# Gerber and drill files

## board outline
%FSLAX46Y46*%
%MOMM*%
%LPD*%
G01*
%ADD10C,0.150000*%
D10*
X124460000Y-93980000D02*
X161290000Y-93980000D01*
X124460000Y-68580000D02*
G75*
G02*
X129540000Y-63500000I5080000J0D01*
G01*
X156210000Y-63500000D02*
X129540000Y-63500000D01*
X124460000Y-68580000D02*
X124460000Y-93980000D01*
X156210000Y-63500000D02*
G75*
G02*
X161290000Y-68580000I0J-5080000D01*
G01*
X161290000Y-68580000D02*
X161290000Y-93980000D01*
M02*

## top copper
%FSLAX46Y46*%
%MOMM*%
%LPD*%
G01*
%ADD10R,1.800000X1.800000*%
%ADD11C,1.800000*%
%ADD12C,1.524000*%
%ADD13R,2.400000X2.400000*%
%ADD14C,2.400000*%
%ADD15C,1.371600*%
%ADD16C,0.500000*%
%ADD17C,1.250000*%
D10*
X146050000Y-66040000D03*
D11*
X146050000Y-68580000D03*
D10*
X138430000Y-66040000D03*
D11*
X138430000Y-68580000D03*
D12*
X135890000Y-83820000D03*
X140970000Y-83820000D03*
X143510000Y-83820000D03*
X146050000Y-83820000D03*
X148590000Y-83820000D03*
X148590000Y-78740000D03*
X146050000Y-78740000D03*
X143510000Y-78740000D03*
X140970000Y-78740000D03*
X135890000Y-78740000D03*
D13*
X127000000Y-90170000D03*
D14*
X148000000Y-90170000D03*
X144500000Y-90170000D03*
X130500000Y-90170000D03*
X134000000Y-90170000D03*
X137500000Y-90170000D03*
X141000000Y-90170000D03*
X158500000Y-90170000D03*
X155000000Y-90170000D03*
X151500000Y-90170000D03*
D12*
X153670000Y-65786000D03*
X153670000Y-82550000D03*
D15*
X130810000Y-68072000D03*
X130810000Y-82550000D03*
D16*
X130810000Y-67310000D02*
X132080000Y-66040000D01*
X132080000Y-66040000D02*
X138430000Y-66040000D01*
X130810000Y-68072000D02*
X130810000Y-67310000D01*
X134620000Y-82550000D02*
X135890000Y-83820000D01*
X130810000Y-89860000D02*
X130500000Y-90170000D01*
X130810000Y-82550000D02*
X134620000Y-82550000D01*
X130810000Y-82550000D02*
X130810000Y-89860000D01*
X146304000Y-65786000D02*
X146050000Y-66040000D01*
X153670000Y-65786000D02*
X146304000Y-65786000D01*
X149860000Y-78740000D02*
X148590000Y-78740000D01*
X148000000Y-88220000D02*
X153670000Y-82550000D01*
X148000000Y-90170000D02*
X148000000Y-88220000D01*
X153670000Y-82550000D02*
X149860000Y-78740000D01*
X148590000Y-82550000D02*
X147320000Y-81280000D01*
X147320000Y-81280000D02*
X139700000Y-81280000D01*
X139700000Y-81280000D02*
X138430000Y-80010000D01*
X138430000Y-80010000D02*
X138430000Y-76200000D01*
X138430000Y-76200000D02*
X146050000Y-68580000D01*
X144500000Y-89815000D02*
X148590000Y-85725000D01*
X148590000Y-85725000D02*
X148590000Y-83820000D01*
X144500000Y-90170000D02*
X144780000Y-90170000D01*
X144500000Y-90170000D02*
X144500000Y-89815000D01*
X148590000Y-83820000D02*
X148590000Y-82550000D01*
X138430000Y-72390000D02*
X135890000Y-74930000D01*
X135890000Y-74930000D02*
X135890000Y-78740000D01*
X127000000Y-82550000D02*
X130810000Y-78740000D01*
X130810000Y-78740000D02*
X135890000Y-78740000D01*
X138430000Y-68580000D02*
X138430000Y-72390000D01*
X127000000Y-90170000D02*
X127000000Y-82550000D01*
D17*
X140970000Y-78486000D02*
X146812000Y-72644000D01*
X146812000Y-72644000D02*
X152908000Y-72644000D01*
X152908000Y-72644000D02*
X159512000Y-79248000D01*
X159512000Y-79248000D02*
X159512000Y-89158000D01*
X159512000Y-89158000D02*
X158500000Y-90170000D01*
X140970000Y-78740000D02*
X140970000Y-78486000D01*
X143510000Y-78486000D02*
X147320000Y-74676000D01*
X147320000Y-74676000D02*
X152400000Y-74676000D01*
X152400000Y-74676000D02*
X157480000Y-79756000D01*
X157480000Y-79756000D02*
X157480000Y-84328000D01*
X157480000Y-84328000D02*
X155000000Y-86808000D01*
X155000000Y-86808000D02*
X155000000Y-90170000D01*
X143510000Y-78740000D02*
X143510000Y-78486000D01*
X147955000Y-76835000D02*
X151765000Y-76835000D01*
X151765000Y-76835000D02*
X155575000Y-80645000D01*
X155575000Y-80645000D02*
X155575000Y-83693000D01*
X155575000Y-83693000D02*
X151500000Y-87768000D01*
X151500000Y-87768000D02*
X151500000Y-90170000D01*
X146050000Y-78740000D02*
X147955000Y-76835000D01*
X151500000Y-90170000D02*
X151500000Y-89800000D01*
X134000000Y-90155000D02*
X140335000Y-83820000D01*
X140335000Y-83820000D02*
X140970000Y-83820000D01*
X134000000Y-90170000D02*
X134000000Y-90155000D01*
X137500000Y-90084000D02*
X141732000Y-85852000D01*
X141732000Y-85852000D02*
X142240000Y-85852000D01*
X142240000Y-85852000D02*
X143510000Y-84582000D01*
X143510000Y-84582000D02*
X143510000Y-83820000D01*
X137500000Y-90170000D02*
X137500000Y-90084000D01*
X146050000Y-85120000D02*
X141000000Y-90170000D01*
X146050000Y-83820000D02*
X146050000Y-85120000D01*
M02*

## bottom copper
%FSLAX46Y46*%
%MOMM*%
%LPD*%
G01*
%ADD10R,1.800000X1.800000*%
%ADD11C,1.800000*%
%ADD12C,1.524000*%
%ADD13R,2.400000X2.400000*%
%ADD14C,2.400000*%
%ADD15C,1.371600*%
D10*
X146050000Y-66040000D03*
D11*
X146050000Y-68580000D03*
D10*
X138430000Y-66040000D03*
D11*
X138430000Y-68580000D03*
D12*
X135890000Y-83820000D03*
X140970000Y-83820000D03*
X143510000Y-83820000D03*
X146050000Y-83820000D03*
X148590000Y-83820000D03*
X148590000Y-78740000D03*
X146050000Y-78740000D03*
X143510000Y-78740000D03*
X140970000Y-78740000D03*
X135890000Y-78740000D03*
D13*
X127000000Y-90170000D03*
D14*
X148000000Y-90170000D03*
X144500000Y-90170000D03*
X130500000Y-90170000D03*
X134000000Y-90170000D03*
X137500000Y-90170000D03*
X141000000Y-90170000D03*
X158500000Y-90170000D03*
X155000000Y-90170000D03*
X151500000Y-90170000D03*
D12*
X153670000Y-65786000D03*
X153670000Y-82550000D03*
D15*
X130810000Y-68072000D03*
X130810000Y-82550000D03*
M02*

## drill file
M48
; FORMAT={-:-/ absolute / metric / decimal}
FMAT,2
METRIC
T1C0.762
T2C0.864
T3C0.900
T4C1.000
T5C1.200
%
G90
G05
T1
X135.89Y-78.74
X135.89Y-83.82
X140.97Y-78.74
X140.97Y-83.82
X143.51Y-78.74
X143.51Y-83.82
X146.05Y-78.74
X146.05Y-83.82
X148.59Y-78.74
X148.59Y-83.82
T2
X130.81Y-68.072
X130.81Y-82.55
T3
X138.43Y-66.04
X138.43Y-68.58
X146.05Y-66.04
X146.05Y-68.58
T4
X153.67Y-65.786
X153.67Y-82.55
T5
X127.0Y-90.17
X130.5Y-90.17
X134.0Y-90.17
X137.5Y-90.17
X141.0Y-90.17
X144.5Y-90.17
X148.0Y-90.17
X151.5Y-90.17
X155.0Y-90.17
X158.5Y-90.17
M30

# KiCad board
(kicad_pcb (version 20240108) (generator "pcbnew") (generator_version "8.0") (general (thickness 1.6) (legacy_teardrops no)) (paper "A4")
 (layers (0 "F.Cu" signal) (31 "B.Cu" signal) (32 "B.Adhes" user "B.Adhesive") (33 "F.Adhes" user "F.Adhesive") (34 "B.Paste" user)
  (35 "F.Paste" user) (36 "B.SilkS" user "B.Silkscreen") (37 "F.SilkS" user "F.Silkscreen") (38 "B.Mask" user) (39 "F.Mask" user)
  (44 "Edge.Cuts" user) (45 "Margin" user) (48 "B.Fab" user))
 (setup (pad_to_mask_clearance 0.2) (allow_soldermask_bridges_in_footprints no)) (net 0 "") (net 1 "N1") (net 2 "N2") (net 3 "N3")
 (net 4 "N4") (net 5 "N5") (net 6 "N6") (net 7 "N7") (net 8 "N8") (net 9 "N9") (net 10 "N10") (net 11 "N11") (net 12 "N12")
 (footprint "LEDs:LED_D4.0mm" (layer "F.Cu") (at 146.05 66.04 -90)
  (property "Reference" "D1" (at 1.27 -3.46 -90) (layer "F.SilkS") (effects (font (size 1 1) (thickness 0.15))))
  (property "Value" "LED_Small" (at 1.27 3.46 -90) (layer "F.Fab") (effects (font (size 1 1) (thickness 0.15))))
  (pad "1" thru_hole rect (at 0 0 270) (size 1.8 1.8) (drill 0.9) (layers "*.Cu" "*.Mask") (remove_unused_layers no) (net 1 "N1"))
  (pad "2" thru_hole circle (at 2.54 0 270) (size 1.8 1.8) (drill 0.9) (layers "*.Cu" "*.Mask") (remove_unused_layers no) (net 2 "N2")))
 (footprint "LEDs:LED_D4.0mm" (layer "F.Cu") (at 138.43 66.04 -90)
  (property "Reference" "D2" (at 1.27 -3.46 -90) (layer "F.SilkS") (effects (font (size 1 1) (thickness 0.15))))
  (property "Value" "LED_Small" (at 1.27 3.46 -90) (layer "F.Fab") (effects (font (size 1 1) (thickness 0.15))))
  (pad "1" thru_hole rect (at 0 0 270) (size 1.8 1.8) (drill 0.9) (layers "*.Cu" "*.Mask") (remove_unused_layers no) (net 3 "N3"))
  (pad "2" thru_hole circle (at 2.54 0 270) (size 1.8 1.8) (drill 0.9) (layers "*.Cu" "*.Mask") (remove_unused_layers no) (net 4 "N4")))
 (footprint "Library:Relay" (layer "F.Cu") (at 135.89 83.82)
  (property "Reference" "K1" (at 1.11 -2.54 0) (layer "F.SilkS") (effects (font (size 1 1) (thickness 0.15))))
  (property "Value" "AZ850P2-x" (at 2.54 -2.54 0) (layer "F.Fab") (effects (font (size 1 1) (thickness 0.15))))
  (pad "1" thru_hole circle (at 0 0) (size 1.524 1.524) (drill 0.762) (layers "*.Cu" "*.Mask") (remove_unused_layers no) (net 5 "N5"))
  (pad "3" thru_hole circle (at 5.08 0) (size 1.524 1.524) (drill 0.762) (layers "*.Cu" "*.Mask") (remove_unused_layers no) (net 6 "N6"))
  (pad "4" thru_hole circle (at 7.62 0) (size 1.524 1.524) (drill 0.762) (layers "*.Cu" "*.Mask") (remove_unused_layers no) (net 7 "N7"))
  (pad "5" thru_hole circle (at 10.16 0) (size 1.524 1.524) (drill 0.762) (layers "*.Cu" "*.Mask") (remove_unused_layers no) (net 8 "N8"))
  (pad "6" thru_hole circle (at 12.7 0) (size 1.524 1.524) (drill 0.762) (layers "*.Cu" "*.Mask") (remove_unused_layers no) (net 2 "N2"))
  (pad "7" thru_hole circle (at 12.7 -5.08) (size 1.524 1.524) (drill 0.762) (layers "*.Cu" "*.Mask") (remove_unused_layers no) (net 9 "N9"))
  (pad "8" thru_hole circle (at 10.16 -5.08) (size 1.524 1.524) (drill 0.762) (layers "*.Cu" "*.Mask") (remove_unused_layers no)
   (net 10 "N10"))
  (pad "9" thru_hole circle (at 7.62 -5.08) (size 1.524 1.524) (drill 0.762) (layers "*.Cu" "*.Mask") (remove_unused_layers no)
   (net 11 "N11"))
  (pad "10" thru_hole circle (at 5.08 -5.08) (size 1.524 1.524) (drill 0.762) (layers "*.Cu" "*.Mask") (remove_unused_layers no)
   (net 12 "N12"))
  (pad "12" thru_hole circle (at 0 -5.08) (size 1.524 1.524) (drill 0.762) (layers "*.Cu" "*.Mask") (remove_unused_layers no) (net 4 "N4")))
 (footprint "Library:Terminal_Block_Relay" (layer "F.Cu") (at 127 90.17)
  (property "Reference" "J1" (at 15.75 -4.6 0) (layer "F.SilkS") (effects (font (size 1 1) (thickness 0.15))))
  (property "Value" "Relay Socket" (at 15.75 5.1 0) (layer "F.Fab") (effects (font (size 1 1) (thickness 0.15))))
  (pad "1" thru_hole rect (at 0 0) (size 2.4 2.4) (drill 1.2) (layers "*.Cu" "*.Mask") (remove_unused_layers no) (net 4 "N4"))
  (pad "2" thru_hole circle (at 21 0) (size 2.4 2.4) (drill 1.2) (layers "*.Cu" "*.Mask") (remove_unused_layers no) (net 9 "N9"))
  (pad "3" thru_hole circle (at 17.5 0) (size 2.4 2.4) (drill 1.2) (layers "*.Cu" "*.Mask") (remove_unused_layers no) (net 2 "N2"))
  (pad "4" thru_hole circle (at 3.5 0) (size 2.4 2.4) (drill 1.2) (layers "*.Cu" "*.Mask") (remove_unused_layers no) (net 5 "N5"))
  (pad "5" thru_hole circle (at 7 0) (size 2.4 2.4) (drill 1.2) (layers "*.Cu" "*.Mask") (remove_unused_layers no) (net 6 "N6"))
  (pad "6" thru_hole circle (at 10.5 0) (size 2.4 2.4) (drill 1.2) (layers "*.Cu" "*.Mask") (remove_unused_layers no) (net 7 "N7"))
  (pad "7" thru_hole circle (at 14 0) (size 2.4 2.4) (drill 1.2) (layers "*.Cu" "*.Mask") (remove_unused_layers no) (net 8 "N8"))
  (pad "8" thru_hole circle (at 31.5 0) (size 2.4 2.4) (drill 1.2) (layers "*.Cu" "*.Mask") (remove_unused_layers no) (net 12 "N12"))
  (pad "9" thru_hole circle (at 28 0) (size 2.4 2.4) (drill 1.2) (layers "*.Cu" "*.Mask") (remove_unused_layers no) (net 11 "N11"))
  (pad "10" thru_hole circle (at 24.5 0) (size 2.4 2.4) (drill 1.2) (layers "*.Cu" "*.Mask") (remove_unused_layers no) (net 10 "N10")))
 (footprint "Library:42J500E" (layer "F.Cu") (at 153.67 82.55 -90)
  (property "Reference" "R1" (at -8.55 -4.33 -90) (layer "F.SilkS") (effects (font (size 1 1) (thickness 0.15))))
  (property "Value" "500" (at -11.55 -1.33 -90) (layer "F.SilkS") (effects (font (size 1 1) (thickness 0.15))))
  (pad "1" thru_hole circle (at -16.764 0 270) (size 1.524 1.524) (drill 1) (layers "*.Cu" "*.Mask") (remove_unused_layers no) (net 1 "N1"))
  (pad "2" thru_hole circle (at 0 0 270) (size 1.524 1.524) (drill 1) (layers "*.Cu" "*.Mask") (remove_unused_layers no) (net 9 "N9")))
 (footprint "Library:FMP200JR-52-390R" (layer "F.Cu") (at 130.81 82.55 -90)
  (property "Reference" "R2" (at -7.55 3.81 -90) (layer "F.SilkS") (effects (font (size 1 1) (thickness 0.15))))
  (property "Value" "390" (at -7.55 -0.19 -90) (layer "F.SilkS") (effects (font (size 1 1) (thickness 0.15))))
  (pad "1" thru_hole circle (at -14.478 0 270) (size 1.3716 1.3716) (drill 0.8636) (layers "*.Cu" "*.Mask") (remove_unused_layers no)
   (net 3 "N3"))
  (pad "2" thru_hole circle (at 0 0 270) (size 1.3716 1.3716) (drill 0.8636) (layers "*.Cu" "*.Mask") (remove_unused_layers no) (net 5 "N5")))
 (gr_line (start 124.46 93.98) (end 161.29 93.98) (stroke (width 0.15) (type solid)) (layer "Edge.Cuts"))
 (gr_arc (start 124.46 68.58) (mid 125.947898 64.987898) (end 129.54 63.5) (stroke (width 0.15) (type solid)) (layer "Edge.Cuts"))
 (gr_line (start 156.21 63.5) (end 129.54 63.5) (stroke (width 0.15) (type solid)) (layer "Edge.Cuts"))
 (gr_line (start 124.46 68.58) (end 124.46 93.98) (stroke (width 0.15) (type solid)) (layer "Edge.Cuts"))
 (gr_arc (start 156.21 63.5) (mid 159.802102 64.987898) (end 161.29 68.58) (stroke (width 0.15) (type solid)) (layer "Edge.Cuts"))
 (gr_line (start 161.29 68.58) (end 161.29 93.98) (stroke (width 0.15) (type solid)) (layer "Edge.Cuts"))
 (segment (start 130.81 67.31) (end 132.08 66.04) (width 0.5) (layer "F.Cu") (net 3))
 (segment (start 132.08 66.04) (end 138.43 66.04) (width 0.5) (layer "F.Cu") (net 3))
 (segment (start 130.81 68.072) (end 130.81 67.31) (width 0.5) (layer "F.Cu") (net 3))
 (segment (start 134.62 82.55) (end 135.89 83.82) (width 0.5) (layer "F.Cu") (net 5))
 (segment (start 130.81 89.86) (end 130.5 90.17) (width 0.5) (layer "F.Cu") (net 5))
 (segment (start 130.81 82.55) (end 134.62 82.55) (width 0.5) (layer "F.Cu") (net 5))
 (segment (start 130.81 82.55) (end 130.81 89.86) (width 0.5) (layer "F.Cu") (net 5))
 (segment (start 146.304 65.786) (end 146.05 66.04) (width 0.5) (layer "F.Cu") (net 1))
 (segment (start 153.67 65.786) (end 146.304 65.786) (width 0.5) (layer "F.Cu") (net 1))
 (segment (start 149.86 78.74) (end 148.59 78.74) (width 0.5) (layer "F.Cu") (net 9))
 (segment (start 148 88.22) (end 153.67 82.55) (width 0.5) (layer "F.Cu") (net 9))
 (segment (start 148 90.17) (end 148 88.22) (width 0.5) (layer "F.Cu") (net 9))
 (segment (start 153.67 82.55) (end 149.86 78.74) (width 0.5) (layer "F.Cu") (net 9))
 (segment (start 148.59 82.55) (end 147.32 81.28) (width 0.5) (layer "F.Cu") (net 2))
 (segment (start 147.32 81.28) (end 139.7 81.28) (width 0.5) (layer "F.Cu") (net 2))
 (segment (start 139.7 81.28) (end 138.43 80.01) (width 0.5) (layer "F.Cu") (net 2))
 (segment (start 138.43 80.01) (end 138.43 76.2) (width 0.5) (layer "F.Cu") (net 2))
 (segment (start 138.43 76.2) (end 146.05 68.58) (width 0.5) (layer "F.Cu") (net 2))
 (segment (start 144.5 89.815) (end 148.59 85.725) (width 0.5) (layer "F.Cu") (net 2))
 (segment (start 148.59 85.725) (end 148.59 83.82) (width 0.5) (layer "F.Cu") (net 2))
 (segment (start 144.5 90.17) (end 144.78 90.17) (width 0.5) (layer "F.Cu") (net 2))
 (segment (start 144.5 90.17) (end 144.5 89.815) (width 0.5) (layer "F.Cu") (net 2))
 (segment (start 148.59 83.82) (end 148.59 82.55) (width 0.5) (layer "F.Cu") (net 2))
 (segment (start 138.43 72.39) (end 135.89 74.93) (width 0.5) (layer "F.Cu") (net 4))
 (segment (start 135.89 74.93) (end 135.89 78.74) (width 0.5) (layer "F.Cu") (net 4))
 (segment (start 127 82.55) (end 130.81 78.74) (width 0.5) (layer "F.Cu") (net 4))
 (segment (start 130.81 78.74) (end 135.89 78.74) (width 0.5) (layer "F.Cu") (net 4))
 (segment (start 138.43 68.58) (end 138.43 72.39) (width 0.5) (layer "F.Cu") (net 4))
 (segment (start 127 90.17) (end 127 82.55) (width 0.5) (layer "F.Cu") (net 4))
 (segment (start 140.97 78.486) (end 146.812 72.644) (width 1.25) (layer "F.Cu") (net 12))
 (segment (start 146.812 72.644) (end 152.908 72.644) (width 1.25) (layer "F.Cu") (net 12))
 (segment (start 152.908 72.644) (end 159.512 79.248) (width 1.25) (layer "F.Cu") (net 12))
 (segment (start 159.512 79.248) (end 159.512 89.158) (width 1.25) (layer "F.Cu") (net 12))
 (segment (start 159.512 89.158) (end 158.5 90.17) (width 1.25) (layer "F.Cu") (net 12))
 (segment (start 140.97 78.74) (end 140.97 78.486) (width 1.25) (layer "F.Cu") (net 12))
 (segment (start 143.51 78.486) (end 147.32 74.676) (width 1.25) (layer "F.Cu") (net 11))
 (segment (start 147.32 74.676) (end 152.4 74.676) (width 1.25) (layer "F.Cu") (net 11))
 (segment (start 152.4 74.676) (end 157.48 79.756) (width 1.25) (layer "F.Cu") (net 11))
 (segment (start 157.48 79.756) (end 157.48 84.328) (width 1.25) (layer "F.Cu") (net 11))
 (segment (start 157.48 84.328) (end 155 86.808) (width 1.25) (layer "F.Cu") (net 11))
 (segment (start 155 86.808) (end 155 90.17) (width 1.25) (layer "F.Cu") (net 11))
 (segment (start 143.51 78.74) (end 143.51 78.486) (width 1.25) (layer "F.Cu") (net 11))
 (segment (start 147.955 76.835) (end 151.765 76.835) (width 1.25) (layer "F.Cu") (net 10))
 (segment (start 151.765 76.835) (end 155.575 80.645) (width 1.25) (layer "F.Cu") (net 10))
 (segment (start 155.575 80.645) (end 155.575 83.693) (width 1.25) (layer "F.Cu") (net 10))
 (segment (start 155.575 83.693) (end 151.5 87.768) (width 1.25) (layer "F.Cu") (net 10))
 (segment (start 151.5 87.768) (end 151.5 90.17) (width 1.25) (layer "F.Cu") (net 10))
 (segment (start 146.05 78.74) (end 147.955 76.835) (width 1.25) (layer "F.Cu") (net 10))
 (segment (start 151.5 90.17) (end 151.5 89.8) (width 1.25) (layer "F.Cu") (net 10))
 (segment (start 134 90.155) (end 140.335 83.82) (width 1.25) (layer "F.Cu") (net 6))
 (segment (start 140.335 83.82) (end 140.97 83.82) (width 1.25) (layer "F.Cu") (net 6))
 (segment (start 134 90.17) (end 134 90.155) (width 1.25) (layer "F.Cu") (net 6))
 (segment (start 137.5 90.084) (end 141.732 85.852) (width 1.25) (layer "F.Cu") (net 7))
 (segment (start 141.732 85.852) (end 142.24 85.852) (width 1.25) (layer "F.Cu") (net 7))
 (segment (start 142.24 85.852) (end 143.51 84.582) (width 1.25) (layer "F.Cu") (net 7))
 (segment (start 143.51 84.582) (end 143.51 83.82) (width 1.25) (layer "F.Cu") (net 7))
 (segment (start 137.5 90.17) (end 137.5 90.084) (width 1.25) (layer "F.Cu") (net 7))
 (segment (start 146.05 85.12) (end 141 90.17) (width 1.25) (layer "F.Cu") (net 8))
 (segment (start 146.05 83.82) (end 146.05 85.12) (width 1.25) (layer "F.Cu") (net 8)))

